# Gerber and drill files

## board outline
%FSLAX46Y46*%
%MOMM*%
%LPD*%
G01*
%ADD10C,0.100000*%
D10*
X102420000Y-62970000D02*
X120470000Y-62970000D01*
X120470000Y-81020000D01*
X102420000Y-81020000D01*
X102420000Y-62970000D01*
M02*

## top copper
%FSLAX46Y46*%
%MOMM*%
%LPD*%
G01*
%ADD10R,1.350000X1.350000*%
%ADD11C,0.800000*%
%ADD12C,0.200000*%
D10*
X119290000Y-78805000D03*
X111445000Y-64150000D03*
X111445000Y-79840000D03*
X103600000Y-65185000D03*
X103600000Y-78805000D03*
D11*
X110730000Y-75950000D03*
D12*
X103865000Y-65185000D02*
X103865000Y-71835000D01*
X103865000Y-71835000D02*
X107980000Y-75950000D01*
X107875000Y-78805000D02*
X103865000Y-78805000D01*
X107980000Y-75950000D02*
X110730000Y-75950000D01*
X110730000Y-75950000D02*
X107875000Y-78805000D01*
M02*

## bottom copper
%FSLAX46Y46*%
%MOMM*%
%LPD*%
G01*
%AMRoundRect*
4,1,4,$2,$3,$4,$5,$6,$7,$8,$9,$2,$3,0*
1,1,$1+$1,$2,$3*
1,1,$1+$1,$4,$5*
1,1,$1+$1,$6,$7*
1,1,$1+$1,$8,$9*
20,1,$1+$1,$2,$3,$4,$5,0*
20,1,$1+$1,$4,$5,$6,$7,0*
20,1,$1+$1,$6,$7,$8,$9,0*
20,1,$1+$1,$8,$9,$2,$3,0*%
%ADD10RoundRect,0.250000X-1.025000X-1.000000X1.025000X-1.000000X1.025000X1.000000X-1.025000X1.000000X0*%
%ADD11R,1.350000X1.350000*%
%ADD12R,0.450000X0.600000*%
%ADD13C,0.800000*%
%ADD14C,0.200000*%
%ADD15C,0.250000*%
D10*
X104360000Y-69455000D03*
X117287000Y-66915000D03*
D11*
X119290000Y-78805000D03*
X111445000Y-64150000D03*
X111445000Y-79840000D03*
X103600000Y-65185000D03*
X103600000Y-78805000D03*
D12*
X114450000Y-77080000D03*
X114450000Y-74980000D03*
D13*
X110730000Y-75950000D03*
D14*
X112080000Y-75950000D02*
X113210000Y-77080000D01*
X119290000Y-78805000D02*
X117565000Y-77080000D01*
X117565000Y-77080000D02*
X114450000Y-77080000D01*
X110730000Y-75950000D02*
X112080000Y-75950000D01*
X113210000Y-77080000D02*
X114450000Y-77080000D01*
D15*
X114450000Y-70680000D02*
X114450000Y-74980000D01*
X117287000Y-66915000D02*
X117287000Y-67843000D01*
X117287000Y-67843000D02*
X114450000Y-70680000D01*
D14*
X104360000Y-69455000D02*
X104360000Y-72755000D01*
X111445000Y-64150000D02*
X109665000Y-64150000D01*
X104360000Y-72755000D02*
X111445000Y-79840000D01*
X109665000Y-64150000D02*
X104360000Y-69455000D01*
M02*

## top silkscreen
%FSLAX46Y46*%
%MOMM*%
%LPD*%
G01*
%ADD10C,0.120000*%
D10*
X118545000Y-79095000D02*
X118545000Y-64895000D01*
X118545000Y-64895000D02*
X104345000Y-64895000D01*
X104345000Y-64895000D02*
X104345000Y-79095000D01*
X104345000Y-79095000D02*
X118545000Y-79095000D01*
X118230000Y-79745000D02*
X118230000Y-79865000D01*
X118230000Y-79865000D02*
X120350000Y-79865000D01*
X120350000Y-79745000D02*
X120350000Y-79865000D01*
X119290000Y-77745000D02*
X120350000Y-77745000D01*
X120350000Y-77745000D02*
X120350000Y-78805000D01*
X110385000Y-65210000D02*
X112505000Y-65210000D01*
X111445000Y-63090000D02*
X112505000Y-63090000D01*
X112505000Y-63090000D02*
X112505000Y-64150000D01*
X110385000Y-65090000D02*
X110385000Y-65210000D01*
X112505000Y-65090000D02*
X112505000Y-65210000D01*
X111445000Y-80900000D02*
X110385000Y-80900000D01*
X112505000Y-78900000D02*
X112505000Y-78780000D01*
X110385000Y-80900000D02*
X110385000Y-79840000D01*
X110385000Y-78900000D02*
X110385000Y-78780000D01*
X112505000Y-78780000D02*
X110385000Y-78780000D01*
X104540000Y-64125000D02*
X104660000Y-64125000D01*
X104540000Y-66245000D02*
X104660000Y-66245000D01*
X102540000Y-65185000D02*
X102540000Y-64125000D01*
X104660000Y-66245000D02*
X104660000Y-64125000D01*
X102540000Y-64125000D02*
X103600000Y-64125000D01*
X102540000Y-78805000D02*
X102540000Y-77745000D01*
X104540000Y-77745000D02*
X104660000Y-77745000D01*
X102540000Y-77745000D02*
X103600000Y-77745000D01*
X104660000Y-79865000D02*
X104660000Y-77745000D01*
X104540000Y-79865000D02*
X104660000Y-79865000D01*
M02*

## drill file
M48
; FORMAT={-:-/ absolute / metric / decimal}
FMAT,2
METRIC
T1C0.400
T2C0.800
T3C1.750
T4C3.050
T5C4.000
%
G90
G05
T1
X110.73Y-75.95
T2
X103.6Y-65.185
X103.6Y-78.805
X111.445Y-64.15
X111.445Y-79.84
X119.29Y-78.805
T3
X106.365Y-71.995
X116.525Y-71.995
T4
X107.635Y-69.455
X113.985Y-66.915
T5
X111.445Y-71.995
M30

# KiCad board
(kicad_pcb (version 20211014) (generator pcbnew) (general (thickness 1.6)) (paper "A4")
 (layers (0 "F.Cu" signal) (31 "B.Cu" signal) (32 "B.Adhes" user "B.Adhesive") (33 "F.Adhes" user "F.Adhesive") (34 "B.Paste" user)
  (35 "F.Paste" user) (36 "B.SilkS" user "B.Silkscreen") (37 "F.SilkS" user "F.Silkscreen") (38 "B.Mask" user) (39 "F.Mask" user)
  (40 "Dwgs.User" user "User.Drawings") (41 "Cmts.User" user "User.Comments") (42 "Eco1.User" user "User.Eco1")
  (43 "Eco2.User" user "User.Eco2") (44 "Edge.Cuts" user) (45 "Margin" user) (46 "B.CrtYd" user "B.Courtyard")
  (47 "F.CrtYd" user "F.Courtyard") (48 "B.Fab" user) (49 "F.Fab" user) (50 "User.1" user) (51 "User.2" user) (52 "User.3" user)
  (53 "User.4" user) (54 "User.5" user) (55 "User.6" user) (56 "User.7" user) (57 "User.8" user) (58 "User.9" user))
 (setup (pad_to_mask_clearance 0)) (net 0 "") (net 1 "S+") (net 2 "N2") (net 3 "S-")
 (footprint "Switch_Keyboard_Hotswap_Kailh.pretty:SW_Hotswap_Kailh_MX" (layer "F.Cu") (at 111.445 71.995)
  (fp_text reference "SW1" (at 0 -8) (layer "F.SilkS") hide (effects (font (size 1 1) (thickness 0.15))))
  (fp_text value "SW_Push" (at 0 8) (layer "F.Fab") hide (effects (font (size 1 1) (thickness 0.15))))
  (fp_line (start 7.1 7.1) (end 7.1 -7.1) (layer "F.SilkS") (width 0.12))
  (fp_line (start 7.1 -7.1) (end -7.1 -7.1) (layer "F.SilkS") (width 0.12))
  (fp_line (start -7.1 -7.1) (end -7.1 7.1) (layer "F.SilkS") (width 0.12))
  (fp_line (start -7.1 7.1) (end 7.1 7.1) (layer "F.SilkS") (width 0.12))
  (pad "" np_thru_hole circle locked (at -5.08 0) (size 1.75 1.75) (drill 1.75) (layers *.Cu *.Mask))
  (pad "" np_thru_hole circle locked (at -3.81 -2.54) (size 3.05 3.05) (drill 3.05) (layers *.Cu *.Mask))
  (pad "" np_thru_hole circle locked (at 2.54 -5.08) (size 3.05 3.05) (drill 3.05) (layers *.Cu *.Mask))
  (pad "" np_thru_hole circle locked (at 5.08 0) (size 1.75 1.75) (drill 1.75) (layers *.Cu *.Mask))
  (pad "" np_thru_hole circle locked (at 0 0) (size 4 4) (drill 4) (layers *.Cu *.Mask))
  (pad "1" smd roundrect locked (at -7.085 -2.54) (size 2.55 2.5) (layers "B.Cu" "B.Paste" "B.Mask") (roundrect_rratio 0.1) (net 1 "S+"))
  (pad "2" smd roundrect locked (at 5.842 -5.08) (size 2.55 2.5) (layers "B.Cu" "B.Paste" "B.Mask") (roundrect_rratio 0.1) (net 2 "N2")))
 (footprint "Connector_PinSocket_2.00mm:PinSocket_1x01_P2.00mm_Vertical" (layer "F.Cu") (at 119.29 78.805)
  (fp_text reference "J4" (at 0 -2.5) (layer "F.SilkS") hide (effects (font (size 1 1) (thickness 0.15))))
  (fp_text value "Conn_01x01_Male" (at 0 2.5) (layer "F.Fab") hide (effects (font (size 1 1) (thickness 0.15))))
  (fp_line (start -1.06 0.94) (end -1.06 1.06) (layer "F.SilkS") (width 0.12))
  (fp_line (start -1.06 1.06) (end 1.06 1.06) (layer "F.SilkS") (width 0.12))
  (fp_line (start 1.06 0.94) (end 1.06 1.06) (layer "F.SilkS") (width 0.12))
  (fp_line (start 0 -1.06) (end 1.06 -1.06) (layer "F.SilkS") (width 0.12))
  (fp_line (start 1.06 -1.06) (end 1.06 0) (layer "F.SilkS") (width 0.12))
  (pad "1" thru_hole rect (at 0 0) (size 1.35 1.35) (drill 0.8) (layers *.Cu *.Mask) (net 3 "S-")))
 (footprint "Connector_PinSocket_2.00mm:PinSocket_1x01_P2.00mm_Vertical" (layer "F.Cu") (at 111.445 64.15)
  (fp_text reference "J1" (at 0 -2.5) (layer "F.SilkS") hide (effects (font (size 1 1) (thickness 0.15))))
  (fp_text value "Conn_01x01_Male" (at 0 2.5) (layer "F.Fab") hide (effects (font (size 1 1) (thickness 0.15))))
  (fp_line (start -1.06 1.06) (end 1.06 1.06) (layer "F.SilkS") (width 0.12))
  (fp_line (start 0 -1.06) (end 1.06 -1.06) (layer "F.SilkS") (width 0.12))
  (fp_line (start 1.06 -1.06) (end 1.06 0) (layer "F.SilkS") (width 0.12))
  (fp_line (start -1.06 0.94) (end -1.06 1.06) (layer "F.SilkS") (width 0.12))
  (fp_line (start 1.06 0.94) (end 1.06 1.06) (layer "F.SilkS") (width 0.12))
  (pad "1" thru_hole rect (at 0 0) (size 1.35 1.35) (drill 0.8) (layers *.Cu *.Mask) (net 1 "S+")))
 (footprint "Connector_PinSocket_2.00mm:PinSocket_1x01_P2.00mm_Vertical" (layer "F.Cu") (at 111.445 79.84 180)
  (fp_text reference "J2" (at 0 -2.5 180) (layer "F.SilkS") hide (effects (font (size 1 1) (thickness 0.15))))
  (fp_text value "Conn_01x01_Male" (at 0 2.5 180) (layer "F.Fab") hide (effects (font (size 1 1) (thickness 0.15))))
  (fp_line (start 0 -1.06) (end 1.06 -1.06) (layer "F.SilkS") (width 0.12))
  (fp_line (start -1.06 0.94) (end -1.06 1.06) (layer "F.SilkS") (width 0.12))
  (fp_line (start 1.06 -1.06) (end 1.06 0) (layer "F.SilkS") (width 0.12))
  (fp_line (start 1.06 0.94) (end 1.06 1.06) (layer "F.SilkS") (width 0.12))
  (fp_line (start -1.06 1.06) (end 1.06 1.06) (layer "F.SilkS") (width 0.12))
  (pad "1" thru_hole rect (at 0 0 180) (size 1.35 1.35) (drill 0.8) (layers *.Cu *.Mask) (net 1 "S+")))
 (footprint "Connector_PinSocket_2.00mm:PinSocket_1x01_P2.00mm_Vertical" (layer "F.Cu") (at 103.6 65.185 90)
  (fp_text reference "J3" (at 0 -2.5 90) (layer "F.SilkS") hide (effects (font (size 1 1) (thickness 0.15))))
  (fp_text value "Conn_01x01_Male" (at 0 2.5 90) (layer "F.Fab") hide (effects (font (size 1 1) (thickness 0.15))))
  (fp_line (start 1.06 0.94) (end 1.06 1.06) (layer "F.SilkS") (width 0.12))
  (fp_line (start -1.06 0.94) (end -1.06 1.06) (layer "F.SilkS") (width 0.12))
  (fp_line (start 0 -1.06) (end 1.06 -1.06) (layer "F.SilkS") (width 0.12))
  (fp_line (start -1.06 1.06) (end 1.06 1.06) (layer "F.SilkS") (width 0.12))
  (fp_line (start 1.06 -1.06) (end 1.06 0) (layer "F.SilkS") (width 0.12))
  (pad "1" thru_hole rect (at 0 0 90) (size 1.35 1.35) (drill 0.8) (layers *.Cu *.Mask) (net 3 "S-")))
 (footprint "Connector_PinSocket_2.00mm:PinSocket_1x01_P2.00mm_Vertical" (layer "F.Cu") (at 103.6 78.805 90)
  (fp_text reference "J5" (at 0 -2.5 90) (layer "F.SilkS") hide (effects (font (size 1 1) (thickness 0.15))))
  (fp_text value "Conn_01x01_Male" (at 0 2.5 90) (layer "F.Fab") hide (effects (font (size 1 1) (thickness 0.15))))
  (fp_line (start 0 -1.06) (end 1.06 -1.06) (layer "F.SilkS") (width 0.12))
  (fp_line (start 1.06 0.94) (end 1.06 1.06) (layer "F.SilkS") (width 0.12))
  (fp_line (start 1.06 -1.06) (end 1.06 0) (layer "F.SilkS") (width 0.12))
  (fp_line (start -1.06 1.06) (end 1.06 1.06) (layer "F.SilkS") (width 0.12))
  (fp_line (start -1.06 0.94) (end -1.06 1.06) (layer "F.SilkS") (width 0.12))
  (pad "1" thru_hole rect (at 0 0 90) (size 1.35 1.35) (drill 0.8) (layers *.Cu *.Mask) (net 3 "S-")))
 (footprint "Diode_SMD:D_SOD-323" (layer "B.Cu") (at 114.45 76.03 90)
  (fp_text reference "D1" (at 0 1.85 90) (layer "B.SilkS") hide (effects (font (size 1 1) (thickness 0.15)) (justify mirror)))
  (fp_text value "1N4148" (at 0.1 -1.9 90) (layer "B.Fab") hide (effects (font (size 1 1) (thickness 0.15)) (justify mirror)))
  (pad "1" smd rect (at -1.05 0 90) (size 0.6 0.45) (layers "B.Cu" "B.Paste" "B.Mask") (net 3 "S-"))
  (pad "2" smd rect (at 1.05 0 90) (size 0.6 0.45) (layers "B.Cu" "B.Paste" "B.Mask") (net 2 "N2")))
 (gr_rect (start 102.42 62.97) (end 120.47 81.02) (layer "Edge.Cuts") (width 0.1) (fill none))
 (segment (start 103.865 65.185) (end 103.865 71.835) (width 0.2) (layer "F.Cu") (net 3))
 (segment (start 103.865 71.835) (end 107.98 75.95) (width 0.2) (layer "F.Cu") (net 3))
 (segment (start 107.875 78.805) (end 103.865 78.805) (width 0.2) (layer "F.Cu") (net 3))
 (segment (start 107.98 75.95) (end 110.73 75.95) (width 0.2) (layer "F.Cu") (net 3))
 (segment (start 110.73 75.95) (end 107.875 78.805) (width 0.2) (layer "F.Cu") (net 3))
 (via (at 110.73 75.95) (size 0.8) (drill 0.4) (layers "F.Cu" "B.Cu") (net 3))
 (segment (start 112.08 75.95) (end 113.21 77.08) (width 0.2) (layer "B.Cu") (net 3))
 (segment (start 119.29 78.805) (end 117.565 77.08) (width 0.2) (layer "B.Cu") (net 3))
 (segment (start 117.565 77.08) (end 114.45 77.08) (width 0.2) (layer "B.Cu") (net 3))
 (segment (start 110.73 75.95) (end 112.08 75.95) (width 0.2) (layer "B.Cu") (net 3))
 (segment (start 113.21 77.08) (end 114.45 77.08) (width 0.2) (layer "B.Cu") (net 3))
 (segment (start 114.45 70.68) (end 114.45 74.98) (width 0.25) (layer "B.Cu") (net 2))
 (segment (start 117.287 66.915) (end 117.287 67.843) (width 0.25) (layer "B.Cu") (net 2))
 (segment (start 117.287 67.843) (end 114.45 70.68) (width 0.25) (layer "B.Cu") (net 2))
 (segment (start 104.36 69.455) (end 104.36 72.755) (width 0.2) (layer "B.Cu") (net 1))
 (segment (start 111.445 64.15) (end 109.665 64.15) (width 0.2) (layer "B.Cu") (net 1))
 (segment (start 104.36 72.755) (end 111.445 79.84) (width 0.2) (layer "B.Cu") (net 1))
 (segment (start 109.665 64.15) (end 104.36 69.455) (width 0.2) (layer "B.Cu") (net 1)))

